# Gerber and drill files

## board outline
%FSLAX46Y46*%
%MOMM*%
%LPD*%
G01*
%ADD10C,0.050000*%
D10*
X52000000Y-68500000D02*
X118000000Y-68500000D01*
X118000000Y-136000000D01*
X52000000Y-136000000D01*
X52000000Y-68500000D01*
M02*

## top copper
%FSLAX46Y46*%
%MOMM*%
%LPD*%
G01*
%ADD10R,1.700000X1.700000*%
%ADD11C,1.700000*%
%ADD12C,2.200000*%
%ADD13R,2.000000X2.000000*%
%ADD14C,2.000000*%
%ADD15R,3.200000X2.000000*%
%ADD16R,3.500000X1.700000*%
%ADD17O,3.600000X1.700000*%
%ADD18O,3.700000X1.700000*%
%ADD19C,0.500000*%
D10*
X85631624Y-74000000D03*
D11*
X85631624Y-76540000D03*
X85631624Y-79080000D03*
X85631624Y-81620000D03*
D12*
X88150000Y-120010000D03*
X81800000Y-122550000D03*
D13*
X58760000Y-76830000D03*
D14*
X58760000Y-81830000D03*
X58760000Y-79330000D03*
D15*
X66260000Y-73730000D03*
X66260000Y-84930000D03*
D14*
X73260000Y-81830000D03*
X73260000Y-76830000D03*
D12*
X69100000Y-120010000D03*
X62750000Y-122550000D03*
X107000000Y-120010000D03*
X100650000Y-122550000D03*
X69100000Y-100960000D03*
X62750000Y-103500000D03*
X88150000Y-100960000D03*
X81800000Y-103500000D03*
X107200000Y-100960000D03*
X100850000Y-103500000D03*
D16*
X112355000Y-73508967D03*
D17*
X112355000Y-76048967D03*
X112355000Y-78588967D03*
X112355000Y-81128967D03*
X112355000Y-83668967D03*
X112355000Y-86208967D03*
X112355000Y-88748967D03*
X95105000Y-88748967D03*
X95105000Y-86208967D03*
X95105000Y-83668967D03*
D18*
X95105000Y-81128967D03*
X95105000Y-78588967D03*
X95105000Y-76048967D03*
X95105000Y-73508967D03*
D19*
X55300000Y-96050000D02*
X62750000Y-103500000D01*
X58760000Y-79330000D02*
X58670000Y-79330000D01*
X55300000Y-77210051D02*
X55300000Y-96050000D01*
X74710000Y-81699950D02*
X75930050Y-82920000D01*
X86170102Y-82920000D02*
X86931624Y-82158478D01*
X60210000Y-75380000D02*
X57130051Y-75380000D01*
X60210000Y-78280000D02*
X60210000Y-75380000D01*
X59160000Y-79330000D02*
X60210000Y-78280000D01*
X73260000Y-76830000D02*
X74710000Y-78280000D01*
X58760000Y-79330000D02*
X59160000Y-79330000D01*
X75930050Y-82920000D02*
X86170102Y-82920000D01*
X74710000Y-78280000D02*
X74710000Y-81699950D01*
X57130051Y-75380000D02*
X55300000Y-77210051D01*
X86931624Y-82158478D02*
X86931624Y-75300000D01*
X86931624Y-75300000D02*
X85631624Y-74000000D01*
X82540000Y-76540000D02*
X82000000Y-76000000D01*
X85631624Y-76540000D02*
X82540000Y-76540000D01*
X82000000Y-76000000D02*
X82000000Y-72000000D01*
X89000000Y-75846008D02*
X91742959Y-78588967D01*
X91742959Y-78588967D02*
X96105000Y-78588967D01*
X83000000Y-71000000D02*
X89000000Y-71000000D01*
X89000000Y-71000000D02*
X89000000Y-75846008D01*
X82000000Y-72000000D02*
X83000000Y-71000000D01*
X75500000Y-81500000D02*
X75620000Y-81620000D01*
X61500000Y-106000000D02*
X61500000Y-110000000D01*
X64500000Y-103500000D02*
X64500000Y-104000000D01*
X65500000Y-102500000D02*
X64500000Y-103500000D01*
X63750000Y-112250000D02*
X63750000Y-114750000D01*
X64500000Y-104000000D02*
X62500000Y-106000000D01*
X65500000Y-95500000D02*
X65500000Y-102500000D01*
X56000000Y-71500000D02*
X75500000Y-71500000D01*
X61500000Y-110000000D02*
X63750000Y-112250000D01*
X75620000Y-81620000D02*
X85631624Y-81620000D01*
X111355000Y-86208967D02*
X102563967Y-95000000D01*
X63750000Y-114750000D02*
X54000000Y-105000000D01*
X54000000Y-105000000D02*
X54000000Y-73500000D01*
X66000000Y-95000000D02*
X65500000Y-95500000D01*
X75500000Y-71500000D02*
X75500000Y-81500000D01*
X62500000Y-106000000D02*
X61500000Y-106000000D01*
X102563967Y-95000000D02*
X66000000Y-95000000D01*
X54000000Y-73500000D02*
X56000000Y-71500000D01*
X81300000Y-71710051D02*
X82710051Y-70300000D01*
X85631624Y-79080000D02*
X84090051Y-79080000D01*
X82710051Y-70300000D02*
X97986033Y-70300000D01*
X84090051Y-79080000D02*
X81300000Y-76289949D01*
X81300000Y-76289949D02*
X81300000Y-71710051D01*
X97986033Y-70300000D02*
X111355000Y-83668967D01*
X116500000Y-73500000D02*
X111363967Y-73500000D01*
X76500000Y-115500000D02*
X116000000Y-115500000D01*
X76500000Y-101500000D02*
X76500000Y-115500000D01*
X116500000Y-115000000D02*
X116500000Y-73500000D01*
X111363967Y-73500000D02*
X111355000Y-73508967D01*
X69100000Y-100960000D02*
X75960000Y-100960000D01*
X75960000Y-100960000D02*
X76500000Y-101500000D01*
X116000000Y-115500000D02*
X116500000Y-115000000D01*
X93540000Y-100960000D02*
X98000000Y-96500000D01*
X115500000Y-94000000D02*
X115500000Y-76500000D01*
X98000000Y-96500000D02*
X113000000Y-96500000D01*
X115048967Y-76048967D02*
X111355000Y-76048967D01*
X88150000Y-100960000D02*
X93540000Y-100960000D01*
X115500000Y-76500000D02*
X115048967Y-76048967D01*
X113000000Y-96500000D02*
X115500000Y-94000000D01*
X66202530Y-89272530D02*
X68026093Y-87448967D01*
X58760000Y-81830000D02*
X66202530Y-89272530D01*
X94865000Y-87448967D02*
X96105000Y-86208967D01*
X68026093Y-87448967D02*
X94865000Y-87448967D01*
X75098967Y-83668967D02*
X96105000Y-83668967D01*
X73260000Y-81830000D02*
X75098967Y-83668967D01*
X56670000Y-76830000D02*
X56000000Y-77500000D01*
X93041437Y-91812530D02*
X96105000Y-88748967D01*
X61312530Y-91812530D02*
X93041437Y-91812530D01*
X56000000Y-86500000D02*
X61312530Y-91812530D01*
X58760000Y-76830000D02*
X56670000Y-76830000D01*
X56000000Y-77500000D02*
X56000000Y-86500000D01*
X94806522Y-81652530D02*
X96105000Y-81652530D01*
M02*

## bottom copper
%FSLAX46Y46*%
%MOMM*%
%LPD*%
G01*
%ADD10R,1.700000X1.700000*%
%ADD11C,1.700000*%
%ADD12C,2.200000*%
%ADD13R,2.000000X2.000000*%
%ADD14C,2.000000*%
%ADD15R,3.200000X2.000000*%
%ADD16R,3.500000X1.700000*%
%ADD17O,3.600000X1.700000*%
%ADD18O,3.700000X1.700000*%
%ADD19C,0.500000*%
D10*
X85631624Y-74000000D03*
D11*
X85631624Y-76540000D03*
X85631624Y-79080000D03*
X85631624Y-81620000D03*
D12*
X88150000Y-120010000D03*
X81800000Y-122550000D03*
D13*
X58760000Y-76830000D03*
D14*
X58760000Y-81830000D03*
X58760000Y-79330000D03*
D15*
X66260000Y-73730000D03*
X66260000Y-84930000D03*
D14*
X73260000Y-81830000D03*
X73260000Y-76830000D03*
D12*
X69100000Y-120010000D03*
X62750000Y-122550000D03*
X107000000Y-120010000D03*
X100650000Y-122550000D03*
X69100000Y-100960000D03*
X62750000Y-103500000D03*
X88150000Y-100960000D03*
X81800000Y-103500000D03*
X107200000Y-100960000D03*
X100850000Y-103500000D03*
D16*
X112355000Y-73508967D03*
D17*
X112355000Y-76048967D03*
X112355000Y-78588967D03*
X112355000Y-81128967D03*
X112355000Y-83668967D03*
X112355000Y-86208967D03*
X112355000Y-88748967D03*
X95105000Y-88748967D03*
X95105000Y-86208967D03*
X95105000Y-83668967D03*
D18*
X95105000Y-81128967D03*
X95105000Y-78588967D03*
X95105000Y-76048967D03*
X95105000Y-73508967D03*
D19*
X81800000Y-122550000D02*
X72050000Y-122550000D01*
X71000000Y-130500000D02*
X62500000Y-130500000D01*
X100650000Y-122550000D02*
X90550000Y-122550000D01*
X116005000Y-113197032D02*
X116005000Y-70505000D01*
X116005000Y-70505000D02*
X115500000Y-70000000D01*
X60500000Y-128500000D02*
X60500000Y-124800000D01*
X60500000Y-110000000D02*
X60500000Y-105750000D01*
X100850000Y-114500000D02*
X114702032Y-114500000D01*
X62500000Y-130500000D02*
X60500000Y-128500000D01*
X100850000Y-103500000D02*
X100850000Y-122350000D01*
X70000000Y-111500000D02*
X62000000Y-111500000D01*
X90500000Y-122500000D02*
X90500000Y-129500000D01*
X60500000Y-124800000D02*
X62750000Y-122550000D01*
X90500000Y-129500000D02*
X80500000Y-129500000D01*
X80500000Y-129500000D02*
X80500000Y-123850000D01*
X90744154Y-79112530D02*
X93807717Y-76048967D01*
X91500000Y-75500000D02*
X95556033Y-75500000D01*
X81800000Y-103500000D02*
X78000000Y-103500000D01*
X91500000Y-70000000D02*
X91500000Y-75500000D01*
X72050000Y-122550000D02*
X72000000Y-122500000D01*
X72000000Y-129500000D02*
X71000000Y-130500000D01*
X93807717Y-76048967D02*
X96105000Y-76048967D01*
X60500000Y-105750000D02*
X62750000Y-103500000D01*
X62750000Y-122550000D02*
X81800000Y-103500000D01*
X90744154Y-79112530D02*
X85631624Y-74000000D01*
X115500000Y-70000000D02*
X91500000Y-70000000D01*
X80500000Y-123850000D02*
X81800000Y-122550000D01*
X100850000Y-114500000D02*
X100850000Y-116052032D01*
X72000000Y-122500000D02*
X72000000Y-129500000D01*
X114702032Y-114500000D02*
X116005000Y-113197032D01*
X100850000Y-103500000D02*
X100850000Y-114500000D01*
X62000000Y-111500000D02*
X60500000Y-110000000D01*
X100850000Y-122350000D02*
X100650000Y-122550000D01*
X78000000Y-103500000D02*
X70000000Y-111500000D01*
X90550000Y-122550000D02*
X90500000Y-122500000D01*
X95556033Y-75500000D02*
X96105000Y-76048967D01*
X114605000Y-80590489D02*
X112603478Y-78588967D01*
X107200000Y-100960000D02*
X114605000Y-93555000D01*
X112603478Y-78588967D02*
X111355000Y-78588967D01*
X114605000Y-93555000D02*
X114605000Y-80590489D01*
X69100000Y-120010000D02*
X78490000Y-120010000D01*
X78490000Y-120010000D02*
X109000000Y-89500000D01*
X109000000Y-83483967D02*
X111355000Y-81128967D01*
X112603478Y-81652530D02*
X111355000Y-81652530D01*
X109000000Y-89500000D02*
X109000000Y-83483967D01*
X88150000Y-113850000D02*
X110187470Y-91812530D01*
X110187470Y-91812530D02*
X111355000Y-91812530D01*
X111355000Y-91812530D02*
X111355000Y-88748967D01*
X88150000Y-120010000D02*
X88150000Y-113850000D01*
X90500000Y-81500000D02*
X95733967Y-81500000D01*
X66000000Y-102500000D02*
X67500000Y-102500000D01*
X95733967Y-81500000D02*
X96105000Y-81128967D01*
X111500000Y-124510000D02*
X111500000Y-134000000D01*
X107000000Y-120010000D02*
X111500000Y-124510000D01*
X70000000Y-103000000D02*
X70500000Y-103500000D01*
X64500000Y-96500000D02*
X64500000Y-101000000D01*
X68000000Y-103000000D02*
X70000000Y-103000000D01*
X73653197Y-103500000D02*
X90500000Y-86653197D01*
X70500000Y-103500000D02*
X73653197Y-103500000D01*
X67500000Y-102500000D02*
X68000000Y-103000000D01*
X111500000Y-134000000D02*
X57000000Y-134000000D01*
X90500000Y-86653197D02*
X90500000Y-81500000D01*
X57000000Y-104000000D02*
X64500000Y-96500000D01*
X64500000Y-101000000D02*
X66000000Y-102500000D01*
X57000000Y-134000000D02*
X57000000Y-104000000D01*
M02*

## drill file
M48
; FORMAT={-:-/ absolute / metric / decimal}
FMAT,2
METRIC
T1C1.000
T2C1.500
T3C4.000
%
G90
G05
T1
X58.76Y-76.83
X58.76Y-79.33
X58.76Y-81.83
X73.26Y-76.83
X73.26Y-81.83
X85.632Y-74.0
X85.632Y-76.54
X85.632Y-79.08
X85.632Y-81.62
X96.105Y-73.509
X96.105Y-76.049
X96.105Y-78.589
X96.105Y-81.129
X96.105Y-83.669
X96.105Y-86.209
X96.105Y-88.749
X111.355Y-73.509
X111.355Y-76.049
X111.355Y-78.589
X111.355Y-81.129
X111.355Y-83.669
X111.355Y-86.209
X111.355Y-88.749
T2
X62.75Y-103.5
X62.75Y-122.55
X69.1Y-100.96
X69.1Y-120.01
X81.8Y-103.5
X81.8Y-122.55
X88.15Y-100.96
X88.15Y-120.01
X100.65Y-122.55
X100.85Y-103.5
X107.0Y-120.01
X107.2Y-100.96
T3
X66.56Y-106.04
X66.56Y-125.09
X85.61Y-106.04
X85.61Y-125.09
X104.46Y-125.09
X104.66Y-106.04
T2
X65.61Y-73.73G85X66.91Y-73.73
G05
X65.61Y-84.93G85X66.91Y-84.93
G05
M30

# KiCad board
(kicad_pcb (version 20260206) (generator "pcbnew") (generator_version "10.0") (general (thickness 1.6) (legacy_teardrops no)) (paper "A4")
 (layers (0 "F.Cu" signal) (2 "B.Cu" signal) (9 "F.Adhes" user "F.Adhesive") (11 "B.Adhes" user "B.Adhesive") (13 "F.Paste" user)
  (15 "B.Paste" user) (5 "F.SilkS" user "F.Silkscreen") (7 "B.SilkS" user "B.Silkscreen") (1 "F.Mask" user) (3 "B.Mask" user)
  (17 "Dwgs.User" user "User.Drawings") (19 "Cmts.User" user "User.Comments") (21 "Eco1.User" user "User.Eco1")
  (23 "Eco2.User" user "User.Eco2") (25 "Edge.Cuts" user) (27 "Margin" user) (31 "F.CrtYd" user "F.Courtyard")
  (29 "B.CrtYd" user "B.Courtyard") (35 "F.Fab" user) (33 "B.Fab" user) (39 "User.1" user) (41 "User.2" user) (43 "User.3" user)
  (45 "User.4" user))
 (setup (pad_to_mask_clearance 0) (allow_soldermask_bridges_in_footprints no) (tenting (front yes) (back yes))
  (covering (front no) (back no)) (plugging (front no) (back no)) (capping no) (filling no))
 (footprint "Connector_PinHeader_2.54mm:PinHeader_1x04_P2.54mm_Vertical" (layer "F.Cu") (at 85.631624 74)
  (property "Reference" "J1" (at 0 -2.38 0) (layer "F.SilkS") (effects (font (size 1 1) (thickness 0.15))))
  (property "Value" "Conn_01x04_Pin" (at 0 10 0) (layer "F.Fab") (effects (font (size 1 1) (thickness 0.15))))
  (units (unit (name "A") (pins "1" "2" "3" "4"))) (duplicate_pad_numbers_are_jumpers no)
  (pad "1" thru_hole rect (at 0 0) (size 1.7 1.7) (drill 1) (layers "*.Cu" "*.Mask") (remove_unused_layers no) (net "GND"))
  (pad "2" thru_hole circle (at 0 2.54) (size 1.7 1.7) (drill 1) (layers "*.Cu" "*.Mask") (remove_unused_layers no) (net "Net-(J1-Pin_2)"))
  (pad "3" thru_hole circle (at 0 5.08) (size 1.7 1.7) (drill 1) (layers "*.Cu" "*.Mask") (remove_unused_layers no) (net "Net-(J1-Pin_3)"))
  (pad "4" thru_hole circle (at 0 7.62) (size 1.7 1.7) (drill 1) (layers "*.Cu" "*.Mask") (remove_unused_layers no) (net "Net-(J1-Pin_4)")))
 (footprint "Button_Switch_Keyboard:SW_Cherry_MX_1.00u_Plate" (layer "F.Cu") (at 88.15 120.01)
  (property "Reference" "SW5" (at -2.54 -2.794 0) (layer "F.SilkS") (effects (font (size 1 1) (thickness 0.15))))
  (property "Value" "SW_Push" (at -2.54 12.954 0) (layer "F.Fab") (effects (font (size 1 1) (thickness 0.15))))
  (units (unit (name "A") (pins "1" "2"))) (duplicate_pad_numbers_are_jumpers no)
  (pad "" np_thru_hole circle (at -2.54 5.08) (size 4 4) (drill 4) (layers "*.Cu" "*.Mask"))
  (pad "1" thru_hole circle (at 0 0) (size 2.2 2.2) (drill 1.5) (layers "*.Cu" "*.Mask") (remove_unused_layers no)
   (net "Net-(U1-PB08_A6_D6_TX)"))
  (pad "2" thru_hole circle (at -6.35 2.54) (size 2.2 2.2) (drill 1.5) (layers "*.Cu" "*.Mask") (remove_unused_layers no) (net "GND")))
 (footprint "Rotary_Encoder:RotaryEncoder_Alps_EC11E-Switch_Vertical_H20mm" (layer "F.Cu") (at 58.76 76.83)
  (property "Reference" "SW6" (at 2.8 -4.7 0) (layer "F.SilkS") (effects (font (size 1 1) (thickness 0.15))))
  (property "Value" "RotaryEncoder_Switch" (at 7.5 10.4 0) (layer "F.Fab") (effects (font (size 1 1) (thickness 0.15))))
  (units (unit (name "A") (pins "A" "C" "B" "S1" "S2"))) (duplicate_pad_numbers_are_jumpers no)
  (pad "A" thru_hole rect (at 0 0) (size 2 2) (drill 1) (layers "*.Cu" "*.Mask") (remove_unused_layers no) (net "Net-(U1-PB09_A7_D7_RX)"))
  (pad "B" thru_hole circle (at 0 5) (size 2 2) (drill 1) (layers "*.Cu" "*.Mask") (remove_unused_layers no) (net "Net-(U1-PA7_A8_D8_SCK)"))
  (pad "C" thru_hole circle (at 0 2.5) (size 2 2) (drill 1) (layers "*.Cu" "*.Mask") (remove_unused_layers no) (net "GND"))
  (pad "MP" thru_hole rect (at 7.5 -3.1) (size 3.2 2) (drill oval 2.8 1.5) (layers "*.Cu" "*.Mask") (remove_unused_layers no))
  (pad "MP" thru_hole rect (at 7.5 8.1) (size 3.2 2) (drill oval 2.8 1.5) (layers "*.Cu" "*.Mask") (remove_unused_layers no))
  (pad "S1" thru_hole circle (at 14.5 5) (size 2 2) (drill 1) (layers "*.Cu" "*.Mask") (remove_unused_layers no)
   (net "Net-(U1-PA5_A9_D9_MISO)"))
  (pad "S2" thru_hole circle (at 14.5 0) (size 2 2) (drill 1) (layers "*.Cu" "*.Mask") (remove_unused_layers no) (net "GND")))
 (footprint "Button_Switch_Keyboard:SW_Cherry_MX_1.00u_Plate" (layer "F.Cu") (at 69.1 120.01)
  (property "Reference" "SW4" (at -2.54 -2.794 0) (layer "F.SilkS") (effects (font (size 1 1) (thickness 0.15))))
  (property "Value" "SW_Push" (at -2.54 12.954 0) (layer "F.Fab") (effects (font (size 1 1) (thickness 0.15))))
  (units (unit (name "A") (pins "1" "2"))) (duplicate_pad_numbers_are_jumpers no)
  (pad "" np_thru_hole circle (at -2.54 5.08) (size 4 4) (drill 4) (layers "*.Cu" "*.Mask"))
  (pad "1" thru_hole circle (at 0 0) (size 2.2 2.2) (drill 1.5) (layers "*.Cu" "*.Mask") (remove_unused_layers no)
   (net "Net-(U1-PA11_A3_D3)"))
  (pad "2" thru_hole circle (at -6.35 2.54) (size 2.2 2.2) (drill 1.5) (layers "*.Cu" "*.Mask") (remove_unused_layers no) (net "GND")))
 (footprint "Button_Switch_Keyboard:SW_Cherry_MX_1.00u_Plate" (layer "F.Cu") (at 107 120.01)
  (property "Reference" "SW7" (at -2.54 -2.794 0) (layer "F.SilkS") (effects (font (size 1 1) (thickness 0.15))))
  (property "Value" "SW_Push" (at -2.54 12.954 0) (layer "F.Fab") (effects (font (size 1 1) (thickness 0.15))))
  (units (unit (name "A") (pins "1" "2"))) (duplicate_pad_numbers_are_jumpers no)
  (pad "" np_thru_hole circle (at -2.54 5.08) (size 4 4) (drill 4) (layers "*.Cu" "*.Mask"))
  (pad "1" thru_hole circle (at 0 0) (size 2.2 2.2) (drill 1.5) (layers "*.Cu" "*.Mask") (remove_unused_layers no)
   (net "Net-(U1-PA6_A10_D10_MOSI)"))
  (pad "2" thru_hole circle (at -6.35 2.54) (size 2.2 2.2) (drill 1.5) (layers "*.Cu" "*.Mask") (remove_unused_layers no) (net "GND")))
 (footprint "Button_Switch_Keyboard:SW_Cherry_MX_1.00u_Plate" (layer "F.Cu") (at 69.1 100.96)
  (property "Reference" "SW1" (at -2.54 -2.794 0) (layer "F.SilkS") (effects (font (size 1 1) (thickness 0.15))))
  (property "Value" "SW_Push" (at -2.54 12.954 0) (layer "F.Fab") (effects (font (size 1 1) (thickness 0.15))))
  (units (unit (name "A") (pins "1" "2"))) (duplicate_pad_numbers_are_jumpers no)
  (pad "" np_thru_hole circle (at -2.54 5.08) (size 4 4) (drill 4) (layers "*.Cu" "*.Mask"))
  (pad "1" thru_hole circle (at 0 0) (size 2.2 2.2) (drill 1.5) (layers "*.Cu" "*.Mask") (remove_unused_layers no)
   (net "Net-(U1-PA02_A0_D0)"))
  (pad "2" thru_hole circle (at -6.35 2.54) (size 2.2 2.2) (drill 1.5) (layers "*.Cu" "*.Mask") (remove_unused_layers no) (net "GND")))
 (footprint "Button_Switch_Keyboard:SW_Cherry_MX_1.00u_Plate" (layer "F.Cu") (at 88.15 100.96)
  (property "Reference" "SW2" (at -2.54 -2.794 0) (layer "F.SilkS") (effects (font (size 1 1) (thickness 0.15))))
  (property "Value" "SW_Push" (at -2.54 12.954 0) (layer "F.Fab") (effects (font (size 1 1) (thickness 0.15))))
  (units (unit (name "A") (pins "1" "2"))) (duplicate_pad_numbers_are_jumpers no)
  (pad "" np_thru_hole circle (at -2.54 5.08) (size 4 4) (drill 4) (layers "*.Cu" "*.Mask"))
  (pad "1" thru_hole circle (at 0 0) (size 2.2 2.2) (drill 1.5) (layers "*.Cu" "*.Mask") (remove_unused_layers no)
   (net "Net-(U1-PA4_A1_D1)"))
  (pad "2" thru_hole circle (at -6.35 2.54) (size 2.2 2.2) (drill 1.5) (layers "*.Cu" "*.Mask") (remove_unused_layers no) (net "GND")))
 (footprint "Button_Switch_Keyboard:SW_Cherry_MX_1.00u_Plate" (layer "F.Cu") (at 107.2 100.96)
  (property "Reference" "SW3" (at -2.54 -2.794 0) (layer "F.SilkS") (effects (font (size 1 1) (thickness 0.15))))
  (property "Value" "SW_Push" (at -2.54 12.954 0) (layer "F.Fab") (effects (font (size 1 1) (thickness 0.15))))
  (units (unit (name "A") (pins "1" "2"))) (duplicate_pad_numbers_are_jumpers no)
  (pad "" np_thru_hole circle (at -2.54 5.08) (size 4 4) (drill 4) (layers "*.Cu" "*.Mask"))
  (pad "1" thru_hole circle (at 0 0) (size 2.2 2.2) (drill 1.5) (layers "*.Cu" "*.Mask") (remove_unused_layers no)
   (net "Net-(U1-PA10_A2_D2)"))
  (pad "2" thru_hole circle (at -6.35 2.54) (size 2.2 2.2) (drill 1.5) (layers "*.Cu" "*.Mask") (remove_unused_layers no) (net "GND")))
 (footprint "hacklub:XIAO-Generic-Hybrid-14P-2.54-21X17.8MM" (layer "B.Cu") (at 103.73 81.128967 180)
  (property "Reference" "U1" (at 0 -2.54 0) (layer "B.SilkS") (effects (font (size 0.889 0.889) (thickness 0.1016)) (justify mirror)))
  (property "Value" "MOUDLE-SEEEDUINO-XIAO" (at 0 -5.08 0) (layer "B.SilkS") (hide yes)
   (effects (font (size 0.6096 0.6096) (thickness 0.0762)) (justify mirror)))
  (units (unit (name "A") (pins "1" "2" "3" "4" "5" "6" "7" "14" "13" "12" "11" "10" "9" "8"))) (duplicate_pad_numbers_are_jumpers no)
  (pad "1" thru_hole rect (at -7.625 7.62 180) (size 3.5 1.7) (drill 1 (offset -1 0)) (layers "*.Cu" "*.Mask") (remove_unused_layers no)
   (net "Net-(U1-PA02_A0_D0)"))
  (pad "2" thru_hole oval (at -7.625 5.08 180) (size 3.6 1.7) (drill 1 (offset -1 0)) (layers "*.Cu" "*.Mask") (remove_unused_layers no)
   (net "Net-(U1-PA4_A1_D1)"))
  (pad "3" thru_hole oval (at -7.625 2.54 180) (size 3.6 1.7) (drill 1 (offset -1 0)) (layers "*.Cu" "*.Mask") (remove_unused_layers no)
   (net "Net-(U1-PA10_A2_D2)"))
  (pad "4" thru_hole oval (at -7.625 0 180) (size 3.6 1.7) (drill 1 (offset -1 0)) (layers "*.Cu" "*.Mask") (remove_unused_layers no)
   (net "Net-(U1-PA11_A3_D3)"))
  (pad "5" thru_hole oval (at -7.625 -2.54 180) (size 3.6 1.7) (drill 1 (offset -1 0)) (layers "*.Cu" "*.Mask") (remove_unused_layers no)
   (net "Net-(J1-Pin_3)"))
  (pad "6" thru_hole oval (at -7.625 -5.08) (size 3.6 1.7) (drill 1 (offset 1 0)) (layers "*.Cu" "*.Mask") (remove_unused_layers no)
   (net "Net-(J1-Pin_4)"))
  (pad "7" thru_hole oval (at -7.625 -7.62 180) (size 3.6 1.7) (drill 1 (offset -1 0)) (layers "*.Cu" "*.Mask") (remove_unused_layers no)
   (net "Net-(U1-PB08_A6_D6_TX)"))
  (pad "8" thru_hole oval (at 7.625 -7.62 180) (size 3.6 1.7) (drill 1 (offset 1 0)) (layers "*.Cu" "*.Mask") (remove_unused_layers no)
   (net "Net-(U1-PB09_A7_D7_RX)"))
  (pad "9" thru_hole oval (at 7.625 -5.08 180) (size 3.6 1.7) (drill 1 (offset 1 0)) (layers "*.Cu" "*.Mask") (remove_unused_layers no)
   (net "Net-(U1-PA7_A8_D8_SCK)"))
  (pad "10" thru_hole oval (at 7.625 -2.54 180) (size 3.6 1.7) (drill 1 (offset 1 0)) (layers "*.Cu" "*.Mask") (remove_unused_layers no)
   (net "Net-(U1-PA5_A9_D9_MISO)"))
  (pad "11" thru_hole oval (at 7.625 0 180) (size 3.7 1.7) (drill 1 (offset 1 0)) (layers "*.Cu" "*.Mask") (remove_unused_layers no)
   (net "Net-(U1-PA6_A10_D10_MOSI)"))
  (pad "12" thru_hole oval (at 7.625 2.54 180) (size 3.7 1.7) (drill 1 (offset 1 0)) (layers "*.Cu" "*.Mask") (remove_unused_layers no)
   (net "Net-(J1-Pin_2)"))
  (pad "13" thru_hole oval (at 7.625 5.08 180) (size 3.7 1.7) (drill 1 (offset 1 0)) (layers "*.Cu" "*.Mask") (remove_unused_layers no)
   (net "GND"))
  (pad "14" thru_hole oval (at 7.625 7.62 180) (size 3.7 1.7) (drill 1 (offset 1 0)) (layers "*.Cu" "*.Mask") (remove_unused_layers no)
   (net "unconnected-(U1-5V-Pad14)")))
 (gr_rect (start 52 68.5) (end 118 136) (stroke (width 0.05) (type default)) (fill no) (layer "Edge.Cuts"))
 (segment (start 55.3 96.05) (end 62.75 103.5) (width 0.5) (layer "F.Cu") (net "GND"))
 (segment (start 58.76 79.33) (end 58.67 79.33) (width 0.5) (layer "F.Cu") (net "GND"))
 (segment (start 55.3 77.210051) (end 55.3 96.05) (width 0.5) (layer "F.Cu") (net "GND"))
 (segment (start 74.71 81.69995) (end 75.93005 82.92) (width 0.5) (layer "F.Cu") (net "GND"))
 (segment (start 86.170102 82.92) (end 86.931624 82.158478) (width 0.5) (layer "F.Cu") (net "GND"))
 (segment (start 60.21 75.38) (end 57.130051 75.38) (width 0.5) (layer "F.Cu") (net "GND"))
 (segment (start 60.21 78.28) (end 60.21 75.38) (width 0.5) (layer "F.Cu") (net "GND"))
 (segment (start 59.16 79.33) (end 60.21 78.28) (width 0.5) (layer "F.Cu") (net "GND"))
 (segment (start 73.26 76.83) (end 74.71 78.28) (width 0.5) (layer "F.Cu") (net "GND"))
 (segment (start 58.76 79.33) (end 59.16 79.33) (width 0.5) (layer "F.Cu") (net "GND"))
 (segment (start 75.93005 82.92) (end 86.170102 82.92) (width 0.5) (layer "F.Cu") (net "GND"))
 (segment (start 74.71 78.28) (end 74.71 81.69995) (width 0.5) (layer "F.Cu") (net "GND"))
 (segment (start 57.130051 75.38) (end 55.3 77.210051) (width 0.5) (layer "F.Cu") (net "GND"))
 (segment (start 86.931624 82.158478) (end 86.931624 75.3) (width 0.5) (layer "F.Cu") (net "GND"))
 (segment (start 86.931624 75.3) (end 85.631624 74) (width 0.5) (layer "F.Cu") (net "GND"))
 (segment (start 81.8 122.55) (end 72.05 122.55) (width 0.5) (layer "B.Cu") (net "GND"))
 (segment (start 71 130.5) (end 62.5 130.5) (width 0.5) (layer "B.Cu") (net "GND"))
 (segment (start 100.65 122.55) (end 90.55 122.55) (width 0.5) (layer "B.Cu") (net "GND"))
 (segment (start 116.005 113.197032) (end 116.005 70.505) (width 0.5) (layer "B.Cu") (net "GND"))
 (segment (start 116.005 70.505) (end 115.5 70) (width 0.5) (layer "B.Cu") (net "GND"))
 (segment (start 60.5 128.5) (end 60.5 124.8) (width 0.5) (layer "B.Cu") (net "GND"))
 (segment (start 60.5 110) (end 60.5 105.75) (width 0.5) (layer "B.Cu") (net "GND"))
 (segment (start 100.85 114.5) (end 114.702032 114.5) (width 0.5) (layer "B.Cu") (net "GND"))
 (segment (start 62.5 130.5) (end 60.5 128.5) (width 0.5) (layer "B.Cu") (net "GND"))
 (segment (start 100.85 103.5) (end 100.85 122.35) (width 0.5) (layer "B.Cu") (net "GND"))
 (segment (start 70 111.5) (end 62 111.5) (width 0.5) (layer "B.Cu") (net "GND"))
 (segment (start 90.5 122.5) (end 90.5 129.5) (width 0.5) (layer "B.Cu") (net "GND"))
 (segment (start 60.5 124.8) (end 62.75 122.55) (width 0.5) (layer "B.Cu") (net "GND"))
 (segment (start 90.5 129.5) (end 80.5 129.5) (width 0.5) (layer "B.Cu") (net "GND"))
 (segment (start 80.5 129.5) (end 80.5 123.85) (width 0.5) (layer "B.Cu") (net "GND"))
 (segment (start 90.744154 79.11253) (end 93.807717 76.048967) (width 0.5) (layer "B.Cu") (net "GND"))
 (segment (start 91.5 75.5) (end 95.556033 75.5) (width 0.5) (layer "B.Cu") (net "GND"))
 (segment (start 81.8 103.5) (end 78 103.5) (width 0.5) (layer "B.Cu") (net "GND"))
 (segment (start 91.5 70) (end 91.5 75.5) (width 0.5) (layer "B.Cu") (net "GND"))
 (segment (start 72.05 122.55) (end 72 122.5) (width 0.5) (layer "B.Cu") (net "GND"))
 (segment (start 72 129.5) (end 71 130.5) (width 0.5) (layer "B.Cu") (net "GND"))
 (segment (start 93.807717 76.048967) (end 96.105 76.048967) (width 0.5) (layer "B.Cu") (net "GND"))
 (segment (start 60.5 105.75) (end 62.75 103.5) (width 0.5) (layer "B.Cu") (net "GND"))
 (segment (start 62.75 122.55) (end 81.8 103.5) (width 0.5) (layer "B.Cu") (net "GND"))
 (segment (start 90.744154 79.11253) (end 85.631624 74) (width 0.5) (layer "B.Cu") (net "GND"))
 (segment (start 115.5 70) (end 91.5 70) (width 0.5) (layer "B.Cu") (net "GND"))
 (segment (start 80.5 123.85) (end 81.8 122.55) (width 0.5) (layer "B.Cu") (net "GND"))
 (segment (start 100.85 114.5) (end 100.85 116.052032) (width 0.5) (layer "B.Cu") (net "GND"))
 (segment (start 72 122.5) (end 72 129.5) (width 0.5) (layer "B.Cu") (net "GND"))
 (segment (start 114.702032 114.5) (end 116.005 113.197032) (width 0.5) (layer "B.Cu") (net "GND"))
 (segment (start 100.85 103.5) (end 100.85 114.5) (width 0.5) (layer "B.Cu") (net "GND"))
 (segment (start 62 111.5) (end 60.5 110) (width 0.5) (layer "B.Cu") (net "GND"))
 (segment (start 100.85 122.35) (end 100.65 122.55) (width 0.5) (layer "B.Cu") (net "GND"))
 (segment (start 78 103.5) (end 70 111.5) (width 0.5) (layer "B.Cu") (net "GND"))
 (segment (start 90.55 122.55) (end 90.5 122.5) (width 0.5) (layer "B.Cu") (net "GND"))
 (segment (start 95.556033 75.5) (end 96.105 76.048967) (width 0.5) (layer "B.Cu") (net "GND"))
 (segment (start 82.54 76.54) (end 82 76) (width 0.5) (layer "F.Cu") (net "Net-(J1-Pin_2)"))
 (segment (start 85.631624 76.54) (end 82.54 76.54) (width 0.5) (layer "F.Cu") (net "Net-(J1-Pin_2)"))
 (segment (start 82 76) (end 82 72) (width 0.5) (layer "F.Cu") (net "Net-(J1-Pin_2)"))
 (segment (start 89 75.846008) (end 91.742959 78.588967) (width 0.5) (layer "F.Cu") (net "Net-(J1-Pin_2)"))
 (segment (start 91.742959 78.588967) (end 96.105 78.588967) (width 0.5) (layer "F.Cu") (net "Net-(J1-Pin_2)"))
 (segment (start 83 71) (end 89 71) (width 0.5) (layer "F.Cu") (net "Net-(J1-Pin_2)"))
 (segment (start 89 71) (end 89 75.846008) (width 0.5) (layer "F.Cu") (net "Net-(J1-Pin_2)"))
 (segment (start 82 72) (end 83 71) (width 0.5) (layer "F.Cu") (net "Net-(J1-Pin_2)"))
 (segment (start 75.5 81.5) (end 75.62 81.62) (width 0.5) (layer "F.Cu") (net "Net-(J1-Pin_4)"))
 (segment (start 61.5 106) (end 61.5 110) (width 0.5) (layer "F.Cu") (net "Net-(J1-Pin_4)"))
 (segment (start 64.5 103.5) (end 64.5 104) (width 0.5) (layer "F.Cu") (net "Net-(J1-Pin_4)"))
 (segment (start 65.5 102.5) (end 64.5 103.5) (width 0.5) (layer "F.Cu") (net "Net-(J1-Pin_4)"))
 (segment (start 63.75 112.25) (end 63.75 114.75) (width 0.5) (layer "F.Cu") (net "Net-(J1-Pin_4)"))
 (segment (start 64.5 104) (end 62.5 106) (width 0.5) (layer "F.Cu") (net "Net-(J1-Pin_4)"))
 (segment (start 65.5 95.5) (end 65.5 102.5) (width 0.5) (layer "F.Cu") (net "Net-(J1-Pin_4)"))
 (segment (start 56 71.5) (end 75.5 71.5) (width 0.5) (layer "F.Cu") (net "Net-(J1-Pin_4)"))
 (segment (start 61.5 110) (end 63.75 112.25) (width 0.5) (layer "F.Cu") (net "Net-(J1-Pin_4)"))
 (segment (start 75.62 81.62) (end 85.631624 81.62) (width 0.5) (layer "F.Cu") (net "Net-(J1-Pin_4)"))
 (segment (start 111.355 86.208967) (end 102.563967 95) (width 0.5) (layer "F.Cu") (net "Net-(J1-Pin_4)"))
 (segment (start 63.75 114.75) (end 54 105) (width 0.5) (layer "F.Cu") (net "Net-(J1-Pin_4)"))
 (segment (start 54 105) (end 54 73.5) (width 0.5) (layer "F.Cu") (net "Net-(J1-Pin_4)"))
 (segment (start 66 95) (end 65.5 95.5) (width 0.5) (layer "F.Cu") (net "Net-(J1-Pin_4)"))
 (segment (start 75.5 71.5) (end 75.5 81.5) (width 0.5) (layer "F.Cu") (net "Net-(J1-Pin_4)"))
 (segment (start 62.5 106) (end 61.5 106) (width 0.5) (layer "F.Cu") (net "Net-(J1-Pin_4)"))
 (segment (start 102.563967 95) (end 66 95) (width 0.5) (layer "F.Cu") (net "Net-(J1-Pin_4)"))
 (segment (start 54 73.5) (end 56 71.5) (width 0.5) (layer "F.Cu") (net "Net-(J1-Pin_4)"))
 (segment (start 81.3 71.710051) (end 82.710051 70.3) (width 0.5) (layer "F.Cu") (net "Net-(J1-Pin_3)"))
 (segment (start 85.631624 79.08) (end 84.090051 79.08) (width 0.5) (layer "F.Cu") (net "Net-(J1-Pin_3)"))
 (segment (start 82.710051 70.3) (end 97.986033 70.3) (width 0.5) (layer "F.Cu") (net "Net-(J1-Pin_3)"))
 (segment (start 84.090051 79.08) (end 81.3 76.289949) (width 0.5) (layer "F.Cu") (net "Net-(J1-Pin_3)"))
 (segment (start 81.3 76.289949) (end 81.3 71.710051) (width 0.5) (layer "F.Cu") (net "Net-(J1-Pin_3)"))
 (segment (start 97.986033 70.3) (end 111.355 83.668967) (width 0.5) (layer "F.Cu") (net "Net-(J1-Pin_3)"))
 (segment (start 116.5 73.5) (end 111.363967 73.5) (width 0.5) (layer "F.Cu") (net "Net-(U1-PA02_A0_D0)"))
 (segment (start 76.5 115.5) (end 116 115.5) (width 0.5) (layer "F.Cu") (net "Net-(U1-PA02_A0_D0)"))
 (segment (start 76.5 101.5) (end 76.5 115.5) (width 0.5) (layer "F.Cu") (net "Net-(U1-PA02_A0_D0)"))
 (segment (start 116.5 115) (end 116.5 73.5) (width 0.5) (layer "F.Cu") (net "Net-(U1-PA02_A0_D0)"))
 (segment (start 111.363967 73.5) (end 111.355 73.508967) (width 0.5) (layer "F.Cu") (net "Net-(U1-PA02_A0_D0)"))
 (segment (start 69.1 100.96) (end 75.96 100.96) (width 0.5) (layer "F.Cu") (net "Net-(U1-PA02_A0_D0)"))
 (segment (start 75.96 100.96) (end 76.5 101.5) (width 0.5) (layer "F.Cu") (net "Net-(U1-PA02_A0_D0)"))
 (segment (start 116 115.5) (end 116.5 115) (width 0.5) (layer "F.Cu") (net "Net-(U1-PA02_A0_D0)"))
 (segment (start 93.54 100.96) (end 98 96.5) (width 0.5) (layer "F.Cu") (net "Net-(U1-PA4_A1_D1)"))
 (segment (start 115.5 94) (end 115.5 76.5) (width 0.5) (layer "F.Cu") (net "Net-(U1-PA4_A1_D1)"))
 (segment (start 98 96.5) (end 113 96.5) (width 0.5) (layer "F.Cu") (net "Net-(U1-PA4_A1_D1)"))
 (segment (start 115.048967 76.048967) (end 111.355 76.048967) (width 0.5) (layer "F.Cu") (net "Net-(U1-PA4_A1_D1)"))
 (segment (start 88.15 100.96) (end 93.54 100.96) (width 0.5) (layer "F.Cu") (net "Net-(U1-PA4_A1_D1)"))
 (segment (start 115.5 76.5) (end 115.048967 76.048967) (width 0.5) (layer "F.Cu") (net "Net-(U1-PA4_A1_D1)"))
 (segment (start 113 96.5) (end 115.5 94) (width 0.5) (layer "F.Cu") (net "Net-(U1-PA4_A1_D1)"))
 (segment (start 114.605 80.590489) (end 112.603478 78.588967) (width 0.5) (layer "B.Cu") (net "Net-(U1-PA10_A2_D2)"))
 (segment (start 107.2 100.96) (end 114.605 93.555) (width 0.5) (layer "B.Cu") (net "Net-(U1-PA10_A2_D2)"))
 (segment (start 112.603478 78.588967) (end 111.355 78.588967) (width 0.5) (layer "B.Cu") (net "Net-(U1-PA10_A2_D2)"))
 (segment (start 114.605 93.555) (end 114.605 80.590489) (width 0.5) (layer "B.Cu") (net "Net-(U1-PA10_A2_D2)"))
 (segment (start 69.1 120.01) (end 78.49 120.01) (width 0.5) (layer "B.Cu") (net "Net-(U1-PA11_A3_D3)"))
 (segment (start 78.49 120.01) (end 109 89.5) (width 0.5) (layer "B.Cu") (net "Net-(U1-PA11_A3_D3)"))
 (segment (start 109 83.483967) (end 111.355 81.128967) (width 0.5) (layer "B.Cu") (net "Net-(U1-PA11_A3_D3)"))
 (segment (start 112.603478 81.65253) (end 111.355 81.65253) (width 0.5) (layer "B.Cu") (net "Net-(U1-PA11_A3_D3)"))
 (segment (start 109 89.5) (end 109 83.483967) (width 0.5) (layer "B.Cu") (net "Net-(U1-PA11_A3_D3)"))
 (segment (start 88.15 113.85) (end 110.18747 91.81253) (width 0.5) (layer "B.Cu") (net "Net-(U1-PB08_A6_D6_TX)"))
 (segment (start 110.18747 91.81253) (end 111.355 91.81253) (width 0.5) (layer "B.Cu") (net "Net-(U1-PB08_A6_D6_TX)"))
 (segment (start 111.355 91.81253) (end 111.355 88.748967) (width 0.5) (layer "B.Cu") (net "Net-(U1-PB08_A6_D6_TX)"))
 (segment (start 88.15 120.01) (end 88.15 113.85) (width 0.5) (layer "B.Cu") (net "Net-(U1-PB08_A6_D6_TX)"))
 (segment (start 66.20253 89.27253) (end 68.026093 87.448967) (width 0.5) (layer "F.Cu") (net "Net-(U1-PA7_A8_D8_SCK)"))
 (segment (start 58.76 81.83) (end 66.20253 89.27253) (width 0.5) (layer "F.Cu") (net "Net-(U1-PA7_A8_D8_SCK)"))
 (segment (start 94.865 87.448967) (end 96.105 86.208967) (width 0.5) (layer "F.Cu") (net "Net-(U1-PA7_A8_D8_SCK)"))
 (segment (start 68.026093 87.448967) (end 94.865 87.448967) (width 0.5) (layer "F.Cu") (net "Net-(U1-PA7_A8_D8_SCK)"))
 (segment (start 75.098967 83.668967) (end 96.105 83.668967) (width 0.5) (layer "F.Cu") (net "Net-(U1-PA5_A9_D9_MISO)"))
 (segment (start 73.26 81.83) (end 75.098967 83.668967) (width 0.5) (layer "F.Cu") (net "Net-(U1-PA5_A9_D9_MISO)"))
 (segment (start 56.67 76.83) (end 56 77.5) (width 0.5) (layer "F.Cu") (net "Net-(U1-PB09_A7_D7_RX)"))
 (segment (start 93.041437 91.81253) (end 96.105 88.748967) (width 0.5) (layer "F.Cu") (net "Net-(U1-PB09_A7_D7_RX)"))
 (segment (start 61.31253 91.81253) (end 93.041437 91.81253) (width 0.5) (layer "F.Cu") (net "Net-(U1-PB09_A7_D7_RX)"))
 (segment (start 56 86.5) (end 61.31253 91.81253) (width 0.5) (layer "F.Cu") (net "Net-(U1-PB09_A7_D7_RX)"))
 (segment (start 58.76 76.83) (end 56.67 76.83) (width 0.5) (layer "F.Cu") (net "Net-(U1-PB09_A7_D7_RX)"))
 (segment (start 56 77.5) (end 56 86.5) (width 0.5) (layer "F.Cu") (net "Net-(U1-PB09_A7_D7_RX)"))
 (segment (start 94.806522 81.65253) (end 96.105 81.65253) (width 0.5) (layer "F.Cu") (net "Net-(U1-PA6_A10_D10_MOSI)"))
 (segment (start 90.5 81.5) (end 95.733967 81.5) (width 0.5) (layer "B.Cu") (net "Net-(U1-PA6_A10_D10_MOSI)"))
 (segment (start 66 102.5) (end 67.5 102.5) (width 0.5) (layer "B.Cu") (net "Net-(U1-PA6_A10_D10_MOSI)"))
 (segment (start 95.733967 81.5) (end 96.105 81.128967) (width 0.5) (layer "B.Cu") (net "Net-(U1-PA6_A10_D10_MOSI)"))
 (segment (start 111.5 124.51) (end 111.5 134) (width 0.5) (layer "B.Cu") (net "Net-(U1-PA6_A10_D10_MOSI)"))
 (segment (start 107 120.01) (end 111.5 124.51) (width 0.5) (layer "B.Cu") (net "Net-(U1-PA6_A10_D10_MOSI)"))
 (segment (start 70 103) (end 70.5 103.5) (width 0.5) (layer "B.Cu") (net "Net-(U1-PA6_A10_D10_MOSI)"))
 (segment (start 64.5 96.5) (end 64.5 101) (width 0.5) (layer "B.Cu") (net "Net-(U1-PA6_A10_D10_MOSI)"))
 (segment (start 68 103) (end 70 103) (width 0.5) (layer "B.Cu") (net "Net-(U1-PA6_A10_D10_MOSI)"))
 (segment (start 73.653197 103.5) (end 90.5 86.653197) (width 0.5) (layer "B.Cu") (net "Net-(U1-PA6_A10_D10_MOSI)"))
 (segment (start 70.5 103.5) (end 73.653197 103.5) (width 0.5) (layer "B.Cu") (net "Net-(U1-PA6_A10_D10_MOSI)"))
 (segment (start 67.5 102.5) (end 68 103) (width 0.5) (layer "B.Cu") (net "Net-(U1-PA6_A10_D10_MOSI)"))
 (segment (start 111.5 134) (end 57 134) (width 0.5) (layer "B.Cu") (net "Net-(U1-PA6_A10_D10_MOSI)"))
 (segment (start 90.5 86.653197) (end 90.5 81.5) (width 0.5) (layer "B.Cu") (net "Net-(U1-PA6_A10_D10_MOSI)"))
 (segment (start 57 104) (end 64.5 96.5) (width 0.5) (layer "B.Cu") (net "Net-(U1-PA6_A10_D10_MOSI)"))
 (segment (start 64.5 101) (end 66 102.5) (width 0.5) (layer "B.Cu") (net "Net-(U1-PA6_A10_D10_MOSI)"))
 (segment (start 57 134) (end 57 104) (width 0.5) (layer "B.Cu") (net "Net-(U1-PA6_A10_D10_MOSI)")))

